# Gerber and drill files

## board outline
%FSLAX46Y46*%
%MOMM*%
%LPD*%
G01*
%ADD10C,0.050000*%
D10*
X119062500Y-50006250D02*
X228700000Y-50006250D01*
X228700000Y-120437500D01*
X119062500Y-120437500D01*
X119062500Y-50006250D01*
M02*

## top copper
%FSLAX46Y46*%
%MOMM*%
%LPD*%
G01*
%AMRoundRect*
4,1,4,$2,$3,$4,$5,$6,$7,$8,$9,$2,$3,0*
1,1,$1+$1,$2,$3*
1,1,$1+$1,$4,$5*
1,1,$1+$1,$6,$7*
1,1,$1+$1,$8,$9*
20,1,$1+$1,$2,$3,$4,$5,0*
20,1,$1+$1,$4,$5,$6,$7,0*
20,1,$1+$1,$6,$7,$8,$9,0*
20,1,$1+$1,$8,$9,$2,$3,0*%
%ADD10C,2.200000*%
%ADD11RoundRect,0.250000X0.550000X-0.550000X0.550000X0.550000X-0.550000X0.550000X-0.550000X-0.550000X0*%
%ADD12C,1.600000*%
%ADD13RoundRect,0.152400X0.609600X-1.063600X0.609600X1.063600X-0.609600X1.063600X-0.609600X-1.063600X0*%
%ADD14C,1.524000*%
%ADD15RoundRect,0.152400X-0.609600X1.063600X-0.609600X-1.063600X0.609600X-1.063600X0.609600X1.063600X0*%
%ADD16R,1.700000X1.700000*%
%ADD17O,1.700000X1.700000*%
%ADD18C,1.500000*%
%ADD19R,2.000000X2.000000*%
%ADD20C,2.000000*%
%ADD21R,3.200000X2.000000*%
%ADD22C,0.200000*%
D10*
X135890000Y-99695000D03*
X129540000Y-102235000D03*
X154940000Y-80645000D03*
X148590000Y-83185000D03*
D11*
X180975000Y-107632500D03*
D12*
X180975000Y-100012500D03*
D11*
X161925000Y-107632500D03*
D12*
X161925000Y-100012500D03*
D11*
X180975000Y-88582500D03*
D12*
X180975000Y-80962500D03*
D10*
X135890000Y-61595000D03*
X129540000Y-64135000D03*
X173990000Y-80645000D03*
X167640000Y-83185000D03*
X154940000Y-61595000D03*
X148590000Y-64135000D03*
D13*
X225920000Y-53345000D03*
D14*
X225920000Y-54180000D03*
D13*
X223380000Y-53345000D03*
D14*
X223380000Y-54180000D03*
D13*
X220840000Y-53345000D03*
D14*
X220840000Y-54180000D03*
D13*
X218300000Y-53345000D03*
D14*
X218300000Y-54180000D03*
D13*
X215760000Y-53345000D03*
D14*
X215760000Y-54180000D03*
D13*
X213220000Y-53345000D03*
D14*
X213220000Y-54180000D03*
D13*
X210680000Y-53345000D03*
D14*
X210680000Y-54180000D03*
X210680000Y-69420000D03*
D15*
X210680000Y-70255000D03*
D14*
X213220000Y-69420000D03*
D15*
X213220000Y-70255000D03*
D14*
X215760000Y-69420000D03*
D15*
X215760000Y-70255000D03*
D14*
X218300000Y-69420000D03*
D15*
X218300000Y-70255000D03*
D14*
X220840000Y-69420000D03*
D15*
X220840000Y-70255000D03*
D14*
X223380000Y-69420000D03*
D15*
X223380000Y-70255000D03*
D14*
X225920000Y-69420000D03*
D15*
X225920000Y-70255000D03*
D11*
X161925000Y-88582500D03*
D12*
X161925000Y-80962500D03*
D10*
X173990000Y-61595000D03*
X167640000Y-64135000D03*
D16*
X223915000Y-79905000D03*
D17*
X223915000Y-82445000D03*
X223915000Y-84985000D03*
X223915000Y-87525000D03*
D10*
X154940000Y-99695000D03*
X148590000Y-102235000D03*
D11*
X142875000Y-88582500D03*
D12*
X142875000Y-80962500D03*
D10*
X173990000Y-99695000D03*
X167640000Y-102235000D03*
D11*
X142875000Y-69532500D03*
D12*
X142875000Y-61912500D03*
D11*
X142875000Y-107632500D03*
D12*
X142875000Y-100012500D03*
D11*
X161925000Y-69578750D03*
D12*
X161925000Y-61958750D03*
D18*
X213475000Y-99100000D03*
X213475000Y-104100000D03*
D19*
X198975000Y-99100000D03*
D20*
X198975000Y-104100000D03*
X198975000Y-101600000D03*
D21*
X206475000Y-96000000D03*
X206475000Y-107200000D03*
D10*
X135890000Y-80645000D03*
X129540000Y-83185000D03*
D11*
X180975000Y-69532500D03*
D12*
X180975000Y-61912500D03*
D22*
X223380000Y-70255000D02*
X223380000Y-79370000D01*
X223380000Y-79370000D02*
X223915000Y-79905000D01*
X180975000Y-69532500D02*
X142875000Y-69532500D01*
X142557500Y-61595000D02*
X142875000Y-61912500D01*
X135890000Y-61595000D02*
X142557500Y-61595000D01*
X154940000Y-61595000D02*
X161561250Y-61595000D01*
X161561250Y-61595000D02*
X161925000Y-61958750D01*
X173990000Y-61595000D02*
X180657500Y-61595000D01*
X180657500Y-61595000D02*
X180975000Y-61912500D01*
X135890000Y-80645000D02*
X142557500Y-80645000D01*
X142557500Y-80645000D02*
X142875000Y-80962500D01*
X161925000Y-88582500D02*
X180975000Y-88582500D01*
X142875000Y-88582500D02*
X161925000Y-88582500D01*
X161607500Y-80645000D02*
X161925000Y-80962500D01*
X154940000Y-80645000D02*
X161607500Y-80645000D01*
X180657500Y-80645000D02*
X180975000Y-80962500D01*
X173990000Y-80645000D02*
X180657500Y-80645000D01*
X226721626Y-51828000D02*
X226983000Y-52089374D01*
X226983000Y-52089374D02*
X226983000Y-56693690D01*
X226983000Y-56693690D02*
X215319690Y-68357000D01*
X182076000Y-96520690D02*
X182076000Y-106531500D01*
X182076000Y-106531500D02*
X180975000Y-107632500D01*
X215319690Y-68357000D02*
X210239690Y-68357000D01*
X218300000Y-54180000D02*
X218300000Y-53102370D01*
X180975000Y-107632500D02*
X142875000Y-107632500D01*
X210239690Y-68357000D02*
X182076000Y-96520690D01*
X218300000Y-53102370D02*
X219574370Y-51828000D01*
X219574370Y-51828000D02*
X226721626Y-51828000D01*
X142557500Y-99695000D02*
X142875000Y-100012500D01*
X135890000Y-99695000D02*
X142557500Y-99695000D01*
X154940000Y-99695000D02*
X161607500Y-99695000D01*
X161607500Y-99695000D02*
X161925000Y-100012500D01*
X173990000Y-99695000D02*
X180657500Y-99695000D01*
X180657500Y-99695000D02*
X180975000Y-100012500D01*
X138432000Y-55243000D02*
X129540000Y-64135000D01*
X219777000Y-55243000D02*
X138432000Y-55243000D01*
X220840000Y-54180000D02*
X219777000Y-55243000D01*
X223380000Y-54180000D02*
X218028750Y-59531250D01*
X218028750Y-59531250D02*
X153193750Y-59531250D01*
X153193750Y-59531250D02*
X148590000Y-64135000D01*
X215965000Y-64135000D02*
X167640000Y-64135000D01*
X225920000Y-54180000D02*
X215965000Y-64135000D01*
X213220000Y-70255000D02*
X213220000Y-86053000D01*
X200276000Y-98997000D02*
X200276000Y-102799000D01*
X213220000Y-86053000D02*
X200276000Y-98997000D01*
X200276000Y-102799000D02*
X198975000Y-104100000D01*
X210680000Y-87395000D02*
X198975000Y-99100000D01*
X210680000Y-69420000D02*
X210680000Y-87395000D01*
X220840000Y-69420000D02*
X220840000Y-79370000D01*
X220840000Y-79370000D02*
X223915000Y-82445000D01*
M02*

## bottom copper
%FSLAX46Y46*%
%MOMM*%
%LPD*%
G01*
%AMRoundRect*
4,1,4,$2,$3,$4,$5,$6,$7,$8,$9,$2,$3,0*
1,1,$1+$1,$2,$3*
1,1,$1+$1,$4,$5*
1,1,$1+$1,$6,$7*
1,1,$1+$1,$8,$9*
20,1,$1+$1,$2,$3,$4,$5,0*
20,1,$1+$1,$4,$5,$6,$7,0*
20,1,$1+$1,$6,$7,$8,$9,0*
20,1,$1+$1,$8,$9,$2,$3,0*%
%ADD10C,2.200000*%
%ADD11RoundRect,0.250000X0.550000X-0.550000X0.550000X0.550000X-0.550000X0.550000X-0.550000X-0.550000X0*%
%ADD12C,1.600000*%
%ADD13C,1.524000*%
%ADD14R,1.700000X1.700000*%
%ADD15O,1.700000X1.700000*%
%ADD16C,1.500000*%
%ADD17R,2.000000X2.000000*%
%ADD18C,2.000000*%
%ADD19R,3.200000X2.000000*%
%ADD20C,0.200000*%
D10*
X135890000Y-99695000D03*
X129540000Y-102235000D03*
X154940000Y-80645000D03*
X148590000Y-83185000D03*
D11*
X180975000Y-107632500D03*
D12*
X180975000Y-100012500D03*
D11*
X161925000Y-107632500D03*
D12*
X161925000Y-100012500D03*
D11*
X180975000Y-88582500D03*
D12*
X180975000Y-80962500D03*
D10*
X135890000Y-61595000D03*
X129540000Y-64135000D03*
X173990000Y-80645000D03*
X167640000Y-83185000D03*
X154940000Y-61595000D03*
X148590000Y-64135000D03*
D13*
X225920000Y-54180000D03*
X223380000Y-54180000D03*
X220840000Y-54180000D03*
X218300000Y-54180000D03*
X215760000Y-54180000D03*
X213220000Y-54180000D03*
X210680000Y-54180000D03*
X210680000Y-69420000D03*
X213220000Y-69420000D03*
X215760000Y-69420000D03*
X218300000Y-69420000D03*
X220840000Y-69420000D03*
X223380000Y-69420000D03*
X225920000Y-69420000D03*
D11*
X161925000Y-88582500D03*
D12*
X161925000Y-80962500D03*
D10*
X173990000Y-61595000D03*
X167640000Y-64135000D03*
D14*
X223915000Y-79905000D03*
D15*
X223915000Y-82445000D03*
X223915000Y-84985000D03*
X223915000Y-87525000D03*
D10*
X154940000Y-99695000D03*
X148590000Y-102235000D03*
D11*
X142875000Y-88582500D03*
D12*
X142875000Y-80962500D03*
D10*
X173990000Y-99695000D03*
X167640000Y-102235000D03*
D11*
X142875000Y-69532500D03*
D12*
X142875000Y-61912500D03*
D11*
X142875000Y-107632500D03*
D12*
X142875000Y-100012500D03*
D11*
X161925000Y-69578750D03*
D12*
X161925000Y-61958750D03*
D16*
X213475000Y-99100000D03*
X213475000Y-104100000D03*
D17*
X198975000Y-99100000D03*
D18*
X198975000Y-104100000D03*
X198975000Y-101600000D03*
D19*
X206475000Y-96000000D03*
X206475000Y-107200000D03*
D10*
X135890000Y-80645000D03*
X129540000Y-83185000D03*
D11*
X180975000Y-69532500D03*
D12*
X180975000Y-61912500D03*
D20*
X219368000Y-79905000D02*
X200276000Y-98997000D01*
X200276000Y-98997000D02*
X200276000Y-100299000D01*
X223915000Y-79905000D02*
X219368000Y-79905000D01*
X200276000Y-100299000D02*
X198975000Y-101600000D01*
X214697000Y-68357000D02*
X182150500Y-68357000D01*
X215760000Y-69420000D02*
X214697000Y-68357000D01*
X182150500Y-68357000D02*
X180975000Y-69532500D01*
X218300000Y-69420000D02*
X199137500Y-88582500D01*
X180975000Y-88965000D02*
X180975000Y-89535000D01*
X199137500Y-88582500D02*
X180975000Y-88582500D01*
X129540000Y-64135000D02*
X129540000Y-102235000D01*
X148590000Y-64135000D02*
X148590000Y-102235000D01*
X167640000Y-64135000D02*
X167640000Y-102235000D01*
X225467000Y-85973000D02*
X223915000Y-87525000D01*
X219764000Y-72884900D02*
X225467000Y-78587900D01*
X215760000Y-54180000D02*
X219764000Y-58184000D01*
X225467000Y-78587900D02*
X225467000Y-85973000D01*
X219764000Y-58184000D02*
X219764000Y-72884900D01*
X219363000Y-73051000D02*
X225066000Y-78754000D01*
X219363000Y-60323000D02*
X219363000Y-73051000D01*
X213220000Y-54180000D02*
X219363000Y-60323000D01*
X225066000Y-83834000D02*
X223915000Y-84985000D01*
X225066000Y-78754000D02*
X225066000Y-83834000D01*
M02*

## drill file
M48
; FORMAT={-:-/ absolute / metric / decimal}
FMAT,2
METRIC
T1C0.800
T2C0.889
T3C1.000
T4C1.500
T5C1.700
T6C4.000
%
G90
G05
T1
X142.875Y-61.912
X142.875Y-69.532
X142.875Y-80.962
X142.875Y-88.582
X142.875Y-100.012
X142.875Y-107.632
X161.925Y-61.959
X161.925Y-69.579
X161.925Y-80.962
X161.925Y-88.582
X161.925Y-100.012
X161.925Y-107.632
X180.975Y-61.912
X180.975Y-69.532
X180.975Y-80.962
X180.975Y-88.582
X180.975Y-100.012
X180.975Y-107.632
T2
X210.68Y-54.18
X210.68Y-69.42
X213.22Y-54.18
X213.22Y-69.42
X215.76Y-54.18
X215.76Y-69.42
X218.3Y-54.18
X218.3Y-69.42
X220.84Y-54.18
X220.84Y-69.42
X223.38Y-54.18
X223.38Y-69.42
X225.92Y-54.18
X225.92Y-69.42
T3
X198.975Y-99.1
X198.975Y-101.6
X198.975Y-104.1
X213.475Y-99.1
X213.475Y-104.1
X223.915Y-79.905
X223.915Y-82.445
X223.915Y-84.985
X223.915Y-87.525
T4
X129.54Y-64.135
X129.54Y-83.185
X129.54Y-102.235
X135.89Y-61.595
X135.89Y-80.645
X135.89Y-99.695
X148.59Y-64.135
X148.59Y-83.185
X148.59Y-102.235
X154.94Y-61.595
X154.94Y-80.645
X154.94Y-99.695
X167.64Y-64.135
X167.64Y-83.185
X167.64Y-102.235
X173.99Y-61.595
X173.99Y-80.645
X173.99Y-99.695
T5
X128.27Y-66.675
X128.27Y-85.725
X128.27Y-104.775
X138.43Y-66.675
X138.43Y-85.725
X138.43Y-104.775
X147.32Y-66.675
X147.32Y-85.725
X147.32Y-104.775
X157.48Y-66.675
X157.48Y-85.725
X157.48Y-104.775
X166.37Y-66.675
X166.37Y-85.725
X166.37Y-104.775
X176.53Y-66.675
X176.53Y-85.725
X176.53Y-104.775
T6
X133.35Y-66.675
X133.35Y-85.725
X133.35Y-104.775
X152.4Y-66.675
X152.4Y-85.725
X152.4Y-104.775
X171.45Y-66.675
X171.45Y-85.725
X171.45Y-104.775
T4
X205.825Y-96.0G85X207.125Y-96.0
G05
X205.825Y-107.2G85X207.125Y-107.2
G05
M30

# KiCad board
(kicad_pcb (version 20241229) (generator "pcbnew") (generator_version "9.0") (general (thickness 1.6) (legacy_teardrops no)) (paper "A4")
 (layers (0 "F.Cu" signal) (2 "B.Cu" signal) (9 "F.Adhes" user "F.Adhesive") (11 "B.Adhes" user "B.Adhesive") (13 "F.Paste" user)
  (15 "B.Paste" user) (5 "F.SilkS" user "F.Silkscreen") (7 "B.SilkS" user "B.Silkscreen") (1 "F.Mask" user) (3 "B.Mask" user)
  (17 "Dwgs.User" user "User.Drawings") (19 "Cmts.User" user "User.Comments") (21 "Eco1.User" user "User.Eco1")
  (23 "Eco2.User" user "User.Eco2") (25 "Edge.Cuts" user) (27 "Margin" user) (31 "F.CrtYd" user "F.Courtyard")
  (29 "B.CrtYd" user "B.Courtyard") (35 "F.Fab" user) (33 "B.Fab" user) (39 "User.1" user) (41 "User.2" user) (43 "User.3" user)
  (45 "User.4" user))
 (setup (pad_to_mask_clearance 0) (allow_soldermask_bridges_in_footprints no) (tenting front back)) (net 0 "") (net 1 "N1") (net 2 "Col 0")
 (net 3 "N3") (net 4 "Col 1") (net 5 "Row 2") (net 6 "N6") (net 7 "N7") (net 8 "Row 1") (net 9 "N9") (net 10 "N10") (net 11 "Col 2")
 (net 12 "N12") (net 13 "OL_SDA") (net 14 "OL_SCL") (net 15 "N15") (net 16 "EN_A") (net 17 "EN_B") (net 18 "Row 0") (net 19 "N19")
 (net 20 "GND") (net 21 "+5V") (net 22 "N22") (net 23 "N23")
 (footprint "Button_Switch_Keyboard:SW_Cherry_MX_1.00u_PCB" (layer "F.Cu") (at 135.89 99.695)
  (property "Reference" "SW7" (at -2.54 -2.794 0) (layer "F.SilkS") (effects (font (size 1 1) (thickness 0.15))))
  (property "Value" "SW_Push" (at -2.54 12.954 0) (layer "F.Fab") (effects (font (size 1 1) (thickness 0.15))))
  (pad "" np_thru_hole circle (at -7.62 5.08) (size 1.7 1.7) (drill 1.7) (layers "*.Cu" "*.Mask"))
  (pad "" np_thru_hole circle (at -2.54 5.08) (size 4 4) (drill 4) (layers "*.Cu" "*.Mask"))
  (pad "" np_thru_hole circle (at 2.54 5.08) (size 1.7 1.7) (drill 1.7) (layers "*.Cu" "*.Mask"))
  (pad "1" thru_hole circle (at 0 0) (size 2.2 2.2) (drill 1.5) (layers "*.Cu" "*.Mask") (remove_unused_layers no) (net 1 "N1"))
  (pad "2" thru_hole circle (at -6.35 2.54) (size 2.2 2.2) (drill 1.5) (layers "*.Cu" "*.Mask") (remove_unused_layers no) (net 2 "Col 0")))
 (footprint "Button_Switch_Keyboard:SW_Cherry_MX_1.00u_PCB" (layer "F.Cu") (at 154.94 80.645)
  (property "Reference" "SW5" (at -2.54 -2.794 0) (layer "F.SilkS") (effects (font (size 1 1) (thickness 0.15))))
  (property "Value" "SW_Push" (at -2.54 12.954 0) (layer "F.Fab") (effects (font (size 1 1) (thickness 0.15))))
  (pad "" np_thru_hole circle (at -7.62 5.08) (size 1.7 1.7) (drill 1.7) (layers "*.Cu" "*.Mask"))
  (pad "" np_thru_hole circle (at -2.54 5.08) (size 4 4) (drill 4) (layers "*.Cu" "*.Mask"))
  (pad "" np_thru_hole circle (at 2.54 5.08) (size 1.7 1.7) (drill 1.7) (layers "*.Cu" "*.Mask"))
  (pad "1" thru_hole circle (at 0 0) (size 2.2 2.2) (drill 1.5) (layers "*.Cu" "*.Mask") (remove_unused_layers no) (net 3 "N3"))
  (pad "2" thru_hole circle (at -6.35 2.54) (size 2.2 2.2) (drill 1.5) (layers "*.Cu" "*.Mask") (remove_unused_layers no) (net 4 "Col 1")))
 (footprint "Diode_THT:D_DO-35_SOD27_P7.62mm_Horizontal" (layer "F.Cu") (at 180.975 107.6325 90)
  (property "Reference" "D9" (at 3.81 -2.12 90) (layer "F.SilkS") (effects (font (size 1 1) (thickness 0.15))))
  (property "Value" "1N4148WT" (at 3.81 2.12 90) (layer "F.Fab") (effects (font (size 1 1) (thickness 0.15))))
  (pad "1" thru_hole roundrect (at 0 0 90) (size 1.6 1.6) (drill 0.8) (layers "*.Cu" "*.Mask") (remove_unused_layers no)
   (roundrect_rratio 0.15625) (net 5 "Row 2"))
  (pad "2" thru_hole circle (at 7.62 0 90) (size 1.6 1.6) (drill 0.8) (layers "*.Cu" "*.Mask") (remove_unused_layers no) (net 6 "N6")))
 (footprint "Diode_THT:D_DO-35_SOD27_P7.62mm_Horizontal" (layer "F.Cu") (at 161.925 107.6325 90)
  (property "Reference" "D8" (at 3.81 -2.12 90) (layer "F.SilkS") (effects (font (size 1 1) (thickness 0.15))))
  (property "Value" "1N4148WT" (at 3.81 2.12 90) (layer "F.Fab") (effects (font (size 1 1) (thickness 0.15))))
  (pad "1" thru_hole roundrect (at 0 0 90) (size 1.6 1.6) (drill 0.8) (layers "*.Cu" "*.Mask") (remove_unused_layers no)
   (roundrect_rratio 0.15625) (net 5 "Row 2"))
  (pad "2" thru_hole circle (at 7.62 0 90) (size 1.6 1.6) (drill 0.8) (layers "*.Cu" "*.Mask") (remove_unused_layers no) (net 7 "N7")))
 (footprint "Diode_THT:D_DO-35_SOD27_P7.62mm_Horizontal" (layer "F.Cu") (at 180.975 88.5825 90)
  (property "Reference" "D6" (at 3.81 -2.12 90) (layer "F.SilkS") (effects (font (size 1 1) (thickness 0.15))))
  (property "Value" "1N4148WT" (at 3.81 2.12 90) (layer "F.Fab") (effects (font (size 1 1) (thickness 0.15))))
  (pad "1" thru_hole roundrect (at 0 0 90) (size 1.6 1.6) (drill 0.8) (layers "*.Cu" "*.Mask") (remove_unused_layers no)
   (roundrect_rratio 0.15625) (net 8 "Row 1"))
  (pad "2" thru_hole circle (at 7.62 0 90) (size 1.6 1.6) (drill 0.8) (layers "*.Cu" "*.Mask") (remove_unused_layers no) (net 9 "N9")))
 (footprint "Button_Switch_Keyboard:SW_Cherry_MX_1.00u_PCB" (layer "F.Cu") (at 135.89 61.595)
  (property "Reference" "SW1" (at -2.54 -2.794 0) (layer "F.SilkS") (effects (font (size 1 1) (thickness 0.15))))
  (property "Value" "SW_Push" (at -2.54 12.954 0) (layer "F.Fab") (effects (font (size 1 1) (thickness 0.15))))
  (pad "" np_thru_hole circle (at -7.62 5.08) (size 1.7 1.7) (drill 1.7) (layers "*.Cu" "*.Mask"))
  (pad "" np_thru_hole circle (at -2.54 5.08) (size 4 4) (drill 4) (layers "*.Cu" "*.Mask"))
  (pad "" np_thru_hole circle (at 2.54 5.08) (size 1.7 1.7) (drill 1.7) (layers "*.Cu" "*.Mask"))
  (pad "1" thru_hole circle (at 0 0) (size 2.2 2.2) (drill 1.5) (layers "*.Cu" "*.Mask") (remove_unused_layers no) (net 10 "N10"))
  (pad "2" thru_hole circle (at -6.35 2.54) (size 2.2 2.2) (drill 1.5) (layers "*.Cu" "*.Mask") (remove_unused_layers no) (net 2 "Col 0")))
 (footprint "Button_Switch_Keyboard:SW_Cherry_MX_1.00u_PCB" (layer "F.Cu") (at 173.99 80.645)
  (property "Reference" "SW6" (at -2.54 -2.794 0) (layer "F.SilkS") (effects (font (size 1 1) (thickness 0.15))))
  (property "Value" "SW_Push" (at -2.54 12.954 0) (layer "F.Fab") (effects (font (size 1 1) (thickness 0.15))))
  (pad "" np_thru_hole circle (at -7.62 5.08) (size 1.7 1.7) (drill 1.7) (layers "*.Cu" "*.Mask"))
  (pad "" np_thru_hole circle (at -2.54 5.08) (size 4 4) (drill 4) (layers "*.Cu" "*.Mask"))
  (pad "" np_thru_hole circle (at 2.54 5.08) (size 1.7 1.7) (drill 1.7) (layers "*.Cu" "*.Mask"))
  (pad "1" thru_hole circle (at 0 0) (size 2.2 2.2) (drill 1.5) (layers "*.Cu" "*.Mask") (remove_unused_layers no) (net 9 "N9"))
  (pad "2" thru_hole circle (at -6.35 2.54) (size 2.2 2.2) (drill 1.5) (layers "*.Cu" "*.Mask") (remove_unused_layers no) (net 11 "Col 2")))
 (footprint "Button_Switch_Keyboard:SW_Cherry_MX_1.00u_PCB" (layer "F.Cu") (at 154.94 61.595)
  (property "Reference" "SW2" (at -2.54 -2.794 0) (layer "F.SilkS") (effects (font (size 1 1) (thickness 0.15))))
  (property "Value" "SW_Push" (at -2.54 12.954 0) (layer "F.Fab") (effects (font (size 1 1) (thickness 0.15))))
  (pad "" np_thru_hole circle (at -7.62 5.08) (size 1.7 1.7) (drill 1.7) (layers "*.Cu" "*.Mask"))
  (pad "" np_thru_hole circle (at -2.54 5.08) (size 4 4) (drill 4) (layers "*.Cu" "*.Mask"))
  (pad "" np_thru_hole circle (at 2.54 5.08) (size 1.7 1.7) (drill 1.7) (layers "*.Cu" "*.Mask"))
  (pad "1" thru_hole circle (at 0 0) (size 2.2 2.2) (drill 1.5) (layers "*.Cu" "*.Mask") (remove_unused_layers no) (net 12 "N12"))
  (pad "2" thru_hole circle (at -6.35 2.54) (size 2.2 2.2) (drill 1.5) (layers "*.Cu" "*.Mask") (remove_unused_layers no) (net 4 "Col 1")))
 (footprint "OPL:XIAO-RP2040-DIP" (layer "F.Cu") (at 218.3 61.8 -90)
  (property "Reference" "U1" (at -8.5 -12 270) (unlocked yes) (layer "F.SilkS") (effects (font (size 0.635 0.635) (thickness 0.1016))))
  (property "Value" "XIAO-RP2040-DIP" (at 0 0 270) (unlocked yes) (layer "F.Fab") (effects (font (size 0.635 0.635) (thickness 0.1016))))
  (pad "1" smd roundrect (at -8.455 -7.62 90) (size 2.432 1.524) (layers "F.Cu" "F.Mask") (roundrect_rratio 0.1) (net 11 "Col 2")
   (thermal_bridge_angle 45))
  (pad "1" thru_hole circle (at -7.62 -7.62 90) (size 1.524 1.524) (drill 0.889) (layers "*.Cu" "*.Mask") (remove_unused_layers no)
   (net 11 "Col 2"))
  (pad "2" smd roundrect (at -8.455 -5.08 90) (size 2.432 1.524) (layers "F.Cu" "F.Mask") (roundrect_rratio 0.1) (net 4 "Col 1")
   (thermal_bridge_angle 45))
  (pad "2" thru_hole circle (at -7.62 -5.08 90) (size 1.524 1.524) (drill 0.889) (layers "*.Cu" "*.Mask") (remove_unused_layers no)
   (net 4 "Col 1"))
  (pad "3" smd roundrect (at -8.455 -2.54 90) (size 2.432 1.524) (layers "F.Cu" "F.Mask") (roundrect_rratio 0.1) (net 2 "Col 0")
   (thermal_bridge_angle 45))
  (pad "3" thru_hole circle (at -7.62 -2.54 90) (size 1.524 1.524) (drill 0.889) (layers "*.Cu" "*.Mask") (remove_unused_layers no)
   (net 2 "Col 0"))
  (pad "4" smd roundrect (at -8.455 0 90) (size 2.432 1.524) (layers "F.Cu" "F.Mask") (roundrect_rratio 0.1) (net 5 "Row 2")
   (thermal_bridge_angle 45))
  (pad "4" thru_hole circle (at -7.62 0 90) (size 1.524 1.524) (drill 0.889) (layers "*.Cu" "*.Mask") (remove_unused_layers no)
   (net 5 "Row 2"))
  (pad "5" smd roundrect (at -8.455 2.54 90) (size 2.432 1.524) (layers "F.Cu" "F.Mask") (roundrect_rratio 0.1) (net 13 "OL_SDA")
   (thermal_bridge_angle 45))
  (pad "5" thru_hole circle (at -7.62 2.54 90) (size 1.524 1.524) (drill 0.889) (layers "*.Cu" "*.Mask") (remove_unused_layers no)
   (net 13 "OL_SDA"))
  (pad "6" smd roundrect (at -8.455 5.08 90) (size 2.432 1.524) (layers "F.Cu" "F.Mask") (roundrect_rratio 0.1) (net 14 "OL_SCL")
   (thermal_bridge_angle 45))
  (pad "6" thru_hole circle (at -7.62 5.08 90) (size 1.524 1.524) (drill 0.889) (layers "*.Cu" "*.Mask") (remove_unused_layers no)
   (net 14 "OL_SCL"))
  (pad "7" smd roundrect (at -8.455 7.62 90) (size 2.432 1.524) (layers "F.Cu" "F.Mask") (roundrect_rratio 0.1) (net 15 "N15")
   (thermal_bridge_angle 45))
  (pad "7" thru_hole circle (at -7.62 7.62 90) (size 1.524 1.524) (drill 0.889) (layers "*.Cu" "*.Mask") (remove_unused_layers no)
   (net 15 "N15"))
  (pad "8" thru_hole circle (at 7.62 7.62 270) (size 1.524 1.524) (drill 0.889) (layers "*.Cu" "*.Mask") (remove_unused_layers no)
   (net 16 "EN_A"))
  (pad "8" smd roundrect (at 8.455 7.62 270) (size 2.432 1.524) (layers "F.Cu" "F.Mask") (roundrect_rratio 0.1) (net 16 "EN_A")
   (thermal_bridge_angle 45))
  (pad "9" thru_hole circle (at 7.62 5.08 270) (size 1.524 1.524) (drill 0.889) (layers "*.Cu" "*.Mask") (remove_unused_layers no)
   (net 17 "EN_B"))
  (pad "9" smd roundrect (at 8.455 5.08 270) (size 2.432 1.524) (layers "F.Cu" "F.Mask") (roundrect_rratio 0.1) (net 17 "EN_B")
   (thermal_bridge_angle 45))
  (pad "10" thru_hole circle (at 7.62 2.54 270) (size 1.524 1.524) (drill 0.889) (layers "*.Cu" "*.Mask") (remove_unused_layers no)
   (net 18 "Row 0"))
  (pad "10" smd roundrect (at 8.455 2.54 270) (size 2.432 1.524) (layers "F.Cu" "F.Mask") (roundrect_rratio 0.1) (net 18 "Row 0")
   (thermal_bridge_angle 45))
  (pad "11" thru_hole circle (at 7.62 0 270) (size 1.524 1.524) (drill 0.889) (layers "*.Cu" "*.Mask") (remove_unused_layers no)
   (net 8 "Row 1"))
  (pad "11" smd roundrect (at 8.455 0 270) (size 2.432 1.524) (layers "F.Cu" "F.Mask") (roundrect_rratio 0.1) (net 8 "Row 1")
   (thermal_bridge_angle 45))
  (pad "12" thru_hole circle (at 7.62 -2.54 270) (size 1.524 1.524) (drill 0.889) (layers "*.Cu" "*.Mask") (remove_unused_layers no)
   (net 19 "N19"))
  (pad "12" smd roundrect (at 8.455 -2.54 270) (size 2.432 1.524) (layers "F.Cu" "F.Mask") (roundrect_rratio 0.1) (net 19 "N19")
   (thermal_bridge_angle 45))
  (pad "13" thru_hole circle (at 7.62 -5.08 270) (size 1.524 1.524) (drill 0.889) (layers "*.Cu" "*.Mask") (remove_unused_layers no)
   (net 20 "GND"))
  (pad "13" smd roundrect (at 8.455 -5.08 270) (size 2.432 1.524) (layers "F.Cu" "F.Mask") (roundrect_rratio 0.1) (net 20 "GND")
   (thermal_bridge_angle 45))
  (pad "14" thru_hole circle (at 7.62 -7.62 270) (size 1.524 1.524) (drill 0.889) (layers "*.Cu" "*.Mask") (remove_unused_layers no)
   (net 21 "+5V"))
  (pad "14" smd roundrect (at 8.455 -7.62 270) (size 2.432 1.524) (layers "F.Cu" "F.Mask") (roundrect_rratio 0.1) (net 21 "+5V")
   (thermal_bridge_angle 45)))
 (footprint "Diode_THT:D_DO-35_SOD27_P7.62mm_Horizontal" (layer "F.Cu") (at 161.925 88.5825 90)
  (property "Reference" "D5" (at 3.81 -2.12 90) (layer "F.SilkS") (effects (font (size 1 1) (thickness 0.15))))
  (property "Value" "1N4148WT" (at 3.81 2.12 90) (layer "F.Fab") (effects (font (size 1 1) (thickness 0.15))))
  (pad "1" thru_hole roundrect (at 0 0 90) (size 1.6 1.6) (drill 0.8) (layers "*.Cu" "*.Mask") (remove_unused_layers no)
   (roundrect_rratio 0.15625) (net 8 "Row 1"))
  (pad "2" thru_hole circle (at 7.62 0 90) (size 1.6 1.6) (drill 0.8) (layers "*.Cu" "*.Mask") (remove_unused_layers no) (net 3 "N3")))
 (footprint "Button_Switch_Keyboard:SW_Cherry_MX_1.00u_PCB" (layer "F.Cu") (at 173.99 61.595)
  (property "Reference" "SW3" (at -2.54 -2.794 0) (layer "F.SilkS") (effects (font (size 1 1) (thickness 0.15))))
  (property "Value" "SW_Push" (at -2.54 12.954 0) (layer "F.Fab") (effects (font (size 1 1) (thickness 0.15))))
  (pad "" np_thru_hole circle (at -7.62 5.08) (size 1.7 1.7) (drill 1.7) (layers "*.Cu" "*.Mask"))
  (pad "" np_thru_hole circle (at -2.54 5.08) (size 4 4) (drill 4) (layers "*.Cu" "*.Mask"))
  (pad "" np_thru_hole circle (at 2.54 5.08) (size 1.7 1.7) (drill 1.7) (layers "*.Cu" "*.Mask"))
  (pad "1" thru_hole circle (at 0 0) (size 2.2 2.2) (drill 1.5) (layers "*.Cu" "*.Mask") (remove_unused_layers no) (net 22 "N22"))
  (pad "2" thru_hole circle (at -6.35 2.54) (size 2.2 2.2) (drill 1.5) (layers "*.Cu" "*.Mask") (remove_unused_layers no) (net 11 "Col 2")))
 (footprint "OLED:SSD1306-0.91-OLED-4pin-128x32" (layer "F.Cu") (at 187.415 77.715)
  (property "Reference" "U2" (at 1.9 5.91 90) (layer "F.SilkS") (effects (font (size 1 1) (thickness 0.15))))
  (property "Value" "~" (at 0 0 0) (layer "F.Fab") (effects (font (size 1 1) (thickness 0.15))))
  (pad "1" thru_hole rect (at 36.5 2.19) (size 1.7 1.7) (drill 1) (layers "*.Cu" "*.Mask") (remove_unused_layers no) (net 20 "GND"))
  (pad "2" thru_hole oval (at 36.5 4.73) (size 1.7 1.7) (drill 1) (layers "*.Cu" "*.Mask") (remove_unused_layers no) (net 19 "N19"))
  (pad "3" thru_hole oval (at 36.5 7.27) (size 1.7 1.7) (drill 1) (layers "*.Cu" "*.Mask") (remove_unused_layers no) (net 14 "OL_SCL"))
  (pad "4" thru_hole oval (at 36.5 9.81) (size 1.7 1.7) (drill 1) (layers "*.Cu" "*.Mask") (remove_unused_layers no) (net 13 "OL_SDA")))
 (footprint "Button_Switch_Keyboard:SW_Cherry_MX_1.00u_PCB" (layer "F.Cu") (at 154.94 99.695)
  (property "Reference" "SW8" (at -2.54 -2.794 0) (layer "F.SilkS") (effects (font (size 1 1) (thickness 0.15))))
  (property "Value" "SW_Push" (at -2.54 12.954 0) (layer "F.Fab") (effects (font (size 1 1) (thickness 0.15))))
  (pad "" np_thru_hole circle (at -7.62 5.08) (size 1.7 1.7) (drill 1.7) (layers "*.Cu" "*.Mask"))
  (pad "" np_thru_hole circle (at -2.54 5.08) (size 4 4) (drill 4) (layers "*.Cu" "*.Mask"))
  (pad "" np_thru_hole circle (at 2.54 5.08) (size 1.7 1.7) (drill 1.7) (layers "*.Cu" "*.Mask"))
  (pad "1" thru_hole circle (at 0 0) (size 2.2 2.2) (drill 1.5) (layers "*.Cu" "*.Mask") (remove_unused_layers no) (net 7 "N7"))
  (pad "2" thru_hole circle (at -6.35 2.54) (size 2.2 2.2) (drill 1.5) (layers "*.Cu" "*.Mask") (remove_unused_layers no) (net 4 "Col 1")))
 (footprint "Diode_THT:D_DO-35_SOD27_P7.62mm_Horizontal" (layer "F.Cu") (at 142.875 88.5825 90)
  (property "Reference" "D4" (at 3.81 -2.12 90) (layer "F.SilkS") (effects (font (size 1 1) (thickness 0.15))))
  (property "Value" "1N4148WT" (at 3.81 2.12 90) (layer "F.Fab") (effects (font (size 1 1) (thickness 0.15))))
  (pad "1" thru_hole roundrect (at 0 0 90) (size 1.6 1.6) (drill 0.8) (layers "*.Cu" "*.Mask") (remove_unused_layers no)
   (roundrect_rratio 0.15625) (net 8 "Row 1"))
  (pad "2" thru_hole circle (at 7.62 0 90) (size 1.6 1.6) (drill 0.8) (layers "*.Cu" "*.Mask") (remove_unused_layers no) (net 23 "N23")))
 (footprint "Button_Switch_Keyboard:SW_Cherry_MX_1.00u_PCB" (layer "F.Cu") (at 173.99 99.695)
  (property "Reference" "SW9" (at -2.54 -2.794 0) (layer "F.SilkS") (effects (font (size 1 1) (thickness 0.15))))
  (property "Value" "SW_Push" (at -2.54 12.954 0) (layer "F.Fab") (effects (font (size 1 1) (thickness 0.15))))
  (pad "" np_thru_hole circle (at -7.62 5.08) (size 1.7 1.7) (drill 1.7) (layers "*.Cu" "*.Mask"))
  (pad "" np_thru_hole circle (at -2.54 5.08) (size 4 4) (drill 4) (layers "*.Cu" "*.Mask"))
  (pad "" np_thru_hole circle (at 2.54 5.08) (size 1.7 1.7) (drill 1.7) (layers "*.Cu" "*.Mask"))
  (pad "1" thru_hole circle (at 0 0) (size 2.2 2.2) (drill 1.5) (layers "*.Cu" "*.Mask") (remove_unused_layers no) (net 6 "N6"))
  (pad "2" thru_hole circle (at -6.35 2.54) (size 2.2 2.2) (drill 1.5) (layers "*.Cu" "*.Mask") (remove_unused_layers no) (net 11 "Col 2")))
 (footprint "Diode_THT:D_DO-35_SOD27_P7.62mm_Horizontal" (layer "F.Cu") (at 142.875 69.5325 90)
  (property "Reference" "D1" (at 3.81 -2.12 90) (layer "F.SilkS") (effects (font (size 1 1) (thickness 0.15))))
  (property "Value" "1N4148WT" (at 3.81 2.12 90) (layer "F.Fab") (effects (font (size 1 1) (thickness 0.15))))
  (pad "1" thru_hole roundrect (at 0 0 90) (size 1.6 1.6) (drill 0.8) (layers "*.Cu" "*.Mask") (remove_unused_layers no)
   (roundrect_rratio 0.15625) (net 18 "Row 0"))
  (pad "2" thru_hole circle (at 7.62 0 90) (size 1.6 1.6) (drill 0.8) (layers "*.Cu" "*.Mask") (remove_unused_layers no) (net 10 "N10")))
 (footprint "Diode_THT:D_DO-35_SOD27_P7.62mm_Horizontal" (layer "F.Cu") (at 142.875 107.6325 90)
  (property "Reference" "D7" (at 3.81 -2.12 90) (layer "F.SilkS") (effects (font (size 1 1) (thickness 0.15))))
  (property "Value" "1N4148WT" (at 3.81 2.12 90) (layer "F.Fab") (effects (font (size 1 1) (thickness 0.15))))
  (pad "1" thru_hole roundrect (at 0 0 90) (size 1.6 1.6) (drill 0.8) (layers "*.Cu" "*.Mask") (remove_unused_layers no)
   (roundrect_rratio 0.15625) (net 5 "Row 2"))
  (pad "2" thru_hole circle (at 7.62 0 90) (size 1.6 1.6) (drill 0.8) (layers "*.Cu" "*.Mask") (remove_unused_layers no) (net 1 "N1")))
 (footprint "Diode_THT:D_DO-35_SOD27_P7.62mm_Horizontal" (layer "F.Cu") (at 161.925 69.57875 90)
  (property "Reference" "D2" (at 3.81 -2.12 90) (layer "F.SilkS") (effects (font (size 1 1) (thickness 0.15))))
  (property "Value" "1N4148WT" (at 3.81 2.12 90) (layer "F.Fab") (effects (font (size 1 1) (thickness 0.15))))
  (pad "1" thru_hole roundrect (at 0 0 90) (size 1.6 1.6) (drill 0.8) (layers "*.Cu" "*.Mask") (remove_unused_layers no)
   (roundrect_rratio 0.15625) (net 18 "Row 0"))
  (pad "2" thru_hole circle (at 7.62 0 90) (size 1.6 1.6) (drill 0.8) (layers "*.Cu" "*.Mask") (remove_unused_layers no) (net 12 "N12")))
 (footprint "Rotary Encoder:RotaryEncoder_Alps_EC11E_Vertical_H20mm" (layer "F.Cu") (at 198.975 99.1)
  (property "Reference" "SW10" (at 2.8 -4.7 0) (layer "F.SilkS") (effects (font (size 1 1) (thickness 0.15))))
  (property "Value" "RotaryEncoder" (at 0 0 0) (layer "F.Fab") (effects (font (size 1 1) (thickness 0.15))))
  (pad "" thru_hole circle (at 14.5 0) (size 1.5 1.5) (drill 1) (layers "*.Cu" "*.Mask") (remove_unused_layers no))
  (pad "" thru_hole circle (at 14.5 5) (size 1.5 1.5) (drill 1) (layers "*.Cu" "*.Mask") (remove_unused_layers no))
  (pad "A" thru_hole rect (at 0 0) (size 2 2) (drill 1) (layers "*.Cu" "*.Mask") (remove_unused_layers no) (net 16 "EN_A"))
  (pad "B" thru_hole circle (at 0 5) (size 2 2) (drill 1) (layers "*.Cu" "*.Mask") (remove_unused_layers no) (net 17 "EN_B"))
  (pad "C" thru_hole circle (at 0 2.5) (size 2 2) (drill 1) (layers "*.Cu" "*.Mask") (remove_unused_layers no) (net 20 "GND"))
  (pad "MP" thru_hole rect (at 7.5 -3.1) (size 3.2 2) (drill oval 2.8 1.5) (layers "*.Cu" "*.Mask") (remove_unused_layers no))
  (pad "MP" thru_hole rect (at 7.5 8.1) (size 3.2 2) (drill oval 2.8 1.5) (layers "*.Cu" "*.Mask") (remove_unused_layers no)))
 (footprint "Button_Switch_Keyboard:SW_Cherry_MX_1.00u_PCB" (layer "F.Cu") (at 135.89 80.645)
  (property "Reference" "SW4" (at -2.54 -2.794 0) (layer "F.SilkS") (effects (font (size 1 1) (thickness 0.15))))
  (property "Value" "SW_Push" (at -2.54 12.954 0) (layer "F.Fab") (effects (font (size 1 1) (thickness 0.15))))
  (pad "" np_thru_hole circle (at -7.62 5.08) (size 1.7 1.7) (drill 1.7) (layers "*.Cu" "*.Mask"))
  (pad "" np_thru_hole circle (at -2.54 5.08) (size 4 4) (drill 4) (layers "*.Cu" "*.Mask"))
  (pad "" np_thru_hole circle (at 2.54 5.08) (size 1.7 1.7) (drill 1.7) (layers "*.Cu" "*.Mask"))
  (pad "1" thru_hole circle (at 0 0) (size 2.2 2.2) (drill 1.5) (layers "*.Cu" "*.Mask") (remove_unused_layers no) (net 23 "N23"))
  (pad "2" thru_hole circle (at -6.35 2.54) (size 2.2 2.2) (drill 1.5) (layers "*.Cu" "*.Mask") (remove_unused_layers no) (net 2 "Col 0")))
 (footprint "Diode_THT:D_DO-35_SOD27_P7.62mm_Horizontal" (layer "F.Cu") (at 180.975 69.5325 90)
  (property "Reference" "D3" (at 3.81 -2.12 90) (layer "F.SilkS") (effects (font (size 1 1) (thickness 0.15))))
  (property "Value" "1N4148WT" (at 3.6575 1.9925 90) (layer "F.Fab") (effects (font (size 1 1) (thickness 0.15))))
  (pad "1" thru_hole roundrect (at 0 0 90) (size 1.6 1.6) (drill 0.8) (layers "*.Cu" "*.Mask") (remove_unused_layers no)
   (roundrect_rratio 0.15625) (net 18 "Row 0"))
  (pad "2" thru_hole circle (at 7.62 0 90) (size 1.6 1.6) (drill 0.8) (layers "*.Cu" "*.Mask") (remove_unused_layers no) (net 22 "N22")))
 (gr_rect (start 119.0625 50.00625) (end 228.7 120.4375) (stroke (width 0.05) (type default)) (fill no) (layer "Edge.Cuts"))
 (segment (start 223.38 70.255) (end 223.38 79.37) (width 0.2) (layer "F.Cu") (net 20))
 (segment (start 223.38 79.37) (end 223.915 79.905) (width 0.2) (layer "F.Cu") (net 20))
 (segment (start 219.368 79.905) (end 200.276 98.997) (width 0.2) (layer "B.Cu") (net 20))
 (segment (start 200.276 98.997) (end 200.276 100.299) (width 0.2) (layer "B.Cu") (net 20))
 (segment (start 223.915 79.905) (end 219.368 79.905) (width 0.2) (layer "B.Cu") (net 20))
 (segment (start 200.276 100.299) (end 198.975 101.6) (width 0.2) (layer "B.Cu") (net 20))
 (segment (start 180.975 69.5325) (end 142.875 69.5325) (width 0.2) (layer "F.Cu") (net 18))
 (segment (start 214.697 68.357) (end 182.1505 68.357) (width 0.2) (layer "B.Cu") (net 18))
 (segment (start 215.76 69.42) (end 214.697 68.357) (width 0.2) (layer "B.Cu") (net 18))
 (segment (start 182.1505 68.357) (end 180.975 69.5325) (width 0.2) (layer "B.Cu") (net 18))
 (segment (start 142.5575 61.595) (end 142.875 61.9125) (width 0.2) (layer "F.Cu") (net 10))
 (segment (start 135.89 61.595) (end 142.5575 61.595) (width 0.2) (layer "F.Cu") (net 10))
 (segment (start 154.94 61.595) (end 161.56125 61.595) (width 0.2) (layer "F.Cu") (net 12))
 (segment (start 161.56125 61.595) (end 161.925 61.95875) (width 0.2) (layer "F.Cu") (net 12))
 (segment (start 173.99 61.595) (end 180.6575 61.595) (width 0.2) (layer "F.Cu") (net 22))
 (segment (start 180.6575 61.595) (end 180.975 61.9125) (width 0.2) (layer "F.Cu") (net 22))
 (segment (start 135.89 80.645) (end 142.5575 80.645) (width 0.2) (layer "F.Cu") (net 23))
 (segment (start 142.5575 80.645) (end 142.875 80.9625) (width 0.2) (layer "F.Cu") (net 23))
 (segment (start 161.925 88.5825) (end 180.975 88.5825) (width 0.2) (layer "F.Cu") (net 8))
 (segment (start 142.875 88.5825) (end 161.925 88.5825) (width 0.2) (layer "F.Cu") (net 8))
 (segment (start 218.3 69.42) (end 199.1375 88.5825) (width 0.2) (layer "B.Cu") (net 8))
 (segment (start 180.975 88.965) (end 180.975 89.535) (width 0.2) (layer "B.Cu") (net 8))
 (segment (start 199.1375 88.5825) (end 180.975 88.5825) (width 0.2) (layer "B.Cu") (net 8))
 (segment (start 161.6075 80.645) (end 161.925 80.9625) (width 0.2) (layer "F.Cu") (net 3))
 (segment (start 154.94 80.645) (end 161.6075 80.645) (width 0.2) (layer "F.Cu") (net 3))
 (segment (start 180.6575 80.645) (end 180.975 80.9625) (width 0.2) (layer "F.Cu") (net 9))
 (segment (start 173.99 80.645) (end 180.6575 80.645) (width 0.2) (layer "F.Cu") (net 9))
 (segment (start 226.721626 51.828) (end 226.983 52.089374) (width 0.2) (layer "F.Cu") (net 5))
 (segment (start 226.983 52.089374) (end 226.983 56.69369) (width 0.2) (layer "F.Cu") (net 5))
 (segment (start 226.983 56.69369) (end 215.31969 68.357) (width 0.2) (layer "F.Cu") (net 5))
 (segment (start 182.076 96.52069) (end 182.076 106.5315) (width 0.2) (layer "F.Cu") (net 5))
 (segment (start 182.076 106.5315) (end 180.975 107.6325) (width 0.2) (layer "F.Cu") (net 5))
 (segment (start 215.31969 68.357) (end 210.23969 68.357) (width 0.2) (layer "F.Cu") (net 5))
 (segment (start 218.3 54.18) (end 218.3 53.10237) (width 0.2) (layer "F.Cu") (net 5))
 (segment (start 180.975 107.6325) (end 142.875 107.6325) (width 0.2) (layer "F.Cu") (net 5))
 (segment (start 210.23969 68.357) (end 182.076 96.52069) (width 0.2) (layer "F.Cu") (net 5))
 (segment (start 218.3 53.10237) (end 219.57437 51.828) (width 0.2) (layer "F.Cu") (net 5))
 (segment (start 219.57437 51.828) (end 226.721626 51.828) (width 0.2) (layer "F.Cu") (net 5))
 (segment (start 142.5575 99.695) (end 142.875 100.0125) (width 0.2) (layer "F.Cu") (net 1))
 (segment (start 135.89 99.695) (end 142.5575 99.695) (width 0.2) (layer "F.Cu") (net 1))
 (segment (start 154.94 99.695) (end 161.6075 99.695) (width 0.2) (layer "F.Cu") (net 7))
 (segment (start 161.6075 99.695) (end 161.925 100.0125) (width 0.2) (layer "F.Cu") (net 7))
 (segment (start 173.99 99.695) (end 180.6575 99.695) (width 0.2) (layer "F.Cu") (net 6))
 (segment (start 180.6575 99.695) (end 180.975 100.0125) (width 0.2) (layer "F.Cu") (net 6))
 (segment (start 138.432 55.243) (end 129.54 64.135) (width 0.2) (layer "F.Cu") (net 2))
 (segment (start 219.777 55.243) (end 138.432 55.243) (width 0.2) (layer "F.Cu") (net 2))
 (segment (start 220.84 54.18) (end 219.777 55.243) (width 0.2) (layer "F.Cu") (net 2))
 (segment (start 129.54 64.135) (end 129.54 102.235) (width 0.2) (layer "B.Cu") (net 2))
 (segment (start 223.38 54.18) (end 218.02875 59.53125) (width 0.2) (layer "F.Cu") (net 4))
 (segment (start 218.02875 59.53125) (end 153.19375 59.53125) (width 0.2) (layer "F.Cu") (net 4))
 (segment (start 153.19375 59.53125) (end 148.59 64.135) (width 0.2) (layer "F.Cu") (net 4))
 (segment (start 148.59 64.135) (end 148.59 102.235) (width 0.2) (layer "B.Cu") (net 4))
 (segment (start 215.965 64.135) (end 167.64 64.135) (width 0.2) (layer "F.Cu") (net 11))
 (segment (start 225.92 54.18) (end 215.965 64.135) (width 0.2) (layer "F.Cu") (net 11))
 (segment (start 167.64 64.135) (end 167.64 102.235) (width 0.2) (layer "B.Cu") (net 11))
 (segment (start 213.22 70.255) (end 213.22 86.053) (width 0.2) (layer "F.Cu") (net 17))
 (segment (start 200.276 98.997) (end 200.276 102.799) (width 0.2) (layer "F.Cu") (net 17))
 (segment (start 213.22 86.053) (end 200.276 98.997) (width 0.2) (layer "F.Cu") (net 17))
 (segment (start 200.276 102.799) (end 198.975 104.1) (width 0.2) (layer "F.Cu") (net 17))
 (segment (start 210.68 87.395) (end 198.975 99.1) (width 0.2) (layer "F.Cu") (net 16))
 (segment (start 210.68 69.42) (end 210.68 87.395) (width 0.2) (layer "F.Cu") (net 16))
 (segment (start 225.467 85.973) (end 223.915 87.525) (width 0.2) (layer "B.Cu") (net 13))
 (segment (start 219.764 72.8849) (end 225.467 78.5879) (width 0.2) (layer "B.Cu") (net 13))
 (segment (start 215.76 54.18) (end 219.764 58.184) (width 0.2) (layer "B.Cu") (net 13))
 (segment (start 225.467 78.5879) (end 225.467 85.973) (width 0.2) (layer "B.Cu") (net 13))
 (segment (start 219.764 58.184) (end 219.764 72.8849) (width 0.2) (layer "B.Cu") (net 13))
 (segment (start 219.363 73.051) (end 225.066 78.754) (width 0.2) (layer "B.Cu") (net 14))
 (segment (start 219.363 60.323) (end 219.363 73.051) (width 0.2) (layer "B.Cu") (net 14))
 (segment (start 213.22 54.18) (end 219.363 60.323) (width 0.2) (layer "B.Cu") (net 14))
 (segment (start 225.066 83.834) (end 223.915 84.985) (width 0.2) (layer "B.Cu") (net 14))
 (segment (start 225.066 78.754) (end 225.066 83.834) (width 0.2) (layer "B.Cu") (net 14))
 (segment (start 220.84 69.42) (end 220.84 79.37) (width 0.2) (layer "F.Cu") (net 19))
 (segment (start 220.84 79.37) (end 223.915 82.445) (width 0.2) (layer "F.Cu") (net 19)))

